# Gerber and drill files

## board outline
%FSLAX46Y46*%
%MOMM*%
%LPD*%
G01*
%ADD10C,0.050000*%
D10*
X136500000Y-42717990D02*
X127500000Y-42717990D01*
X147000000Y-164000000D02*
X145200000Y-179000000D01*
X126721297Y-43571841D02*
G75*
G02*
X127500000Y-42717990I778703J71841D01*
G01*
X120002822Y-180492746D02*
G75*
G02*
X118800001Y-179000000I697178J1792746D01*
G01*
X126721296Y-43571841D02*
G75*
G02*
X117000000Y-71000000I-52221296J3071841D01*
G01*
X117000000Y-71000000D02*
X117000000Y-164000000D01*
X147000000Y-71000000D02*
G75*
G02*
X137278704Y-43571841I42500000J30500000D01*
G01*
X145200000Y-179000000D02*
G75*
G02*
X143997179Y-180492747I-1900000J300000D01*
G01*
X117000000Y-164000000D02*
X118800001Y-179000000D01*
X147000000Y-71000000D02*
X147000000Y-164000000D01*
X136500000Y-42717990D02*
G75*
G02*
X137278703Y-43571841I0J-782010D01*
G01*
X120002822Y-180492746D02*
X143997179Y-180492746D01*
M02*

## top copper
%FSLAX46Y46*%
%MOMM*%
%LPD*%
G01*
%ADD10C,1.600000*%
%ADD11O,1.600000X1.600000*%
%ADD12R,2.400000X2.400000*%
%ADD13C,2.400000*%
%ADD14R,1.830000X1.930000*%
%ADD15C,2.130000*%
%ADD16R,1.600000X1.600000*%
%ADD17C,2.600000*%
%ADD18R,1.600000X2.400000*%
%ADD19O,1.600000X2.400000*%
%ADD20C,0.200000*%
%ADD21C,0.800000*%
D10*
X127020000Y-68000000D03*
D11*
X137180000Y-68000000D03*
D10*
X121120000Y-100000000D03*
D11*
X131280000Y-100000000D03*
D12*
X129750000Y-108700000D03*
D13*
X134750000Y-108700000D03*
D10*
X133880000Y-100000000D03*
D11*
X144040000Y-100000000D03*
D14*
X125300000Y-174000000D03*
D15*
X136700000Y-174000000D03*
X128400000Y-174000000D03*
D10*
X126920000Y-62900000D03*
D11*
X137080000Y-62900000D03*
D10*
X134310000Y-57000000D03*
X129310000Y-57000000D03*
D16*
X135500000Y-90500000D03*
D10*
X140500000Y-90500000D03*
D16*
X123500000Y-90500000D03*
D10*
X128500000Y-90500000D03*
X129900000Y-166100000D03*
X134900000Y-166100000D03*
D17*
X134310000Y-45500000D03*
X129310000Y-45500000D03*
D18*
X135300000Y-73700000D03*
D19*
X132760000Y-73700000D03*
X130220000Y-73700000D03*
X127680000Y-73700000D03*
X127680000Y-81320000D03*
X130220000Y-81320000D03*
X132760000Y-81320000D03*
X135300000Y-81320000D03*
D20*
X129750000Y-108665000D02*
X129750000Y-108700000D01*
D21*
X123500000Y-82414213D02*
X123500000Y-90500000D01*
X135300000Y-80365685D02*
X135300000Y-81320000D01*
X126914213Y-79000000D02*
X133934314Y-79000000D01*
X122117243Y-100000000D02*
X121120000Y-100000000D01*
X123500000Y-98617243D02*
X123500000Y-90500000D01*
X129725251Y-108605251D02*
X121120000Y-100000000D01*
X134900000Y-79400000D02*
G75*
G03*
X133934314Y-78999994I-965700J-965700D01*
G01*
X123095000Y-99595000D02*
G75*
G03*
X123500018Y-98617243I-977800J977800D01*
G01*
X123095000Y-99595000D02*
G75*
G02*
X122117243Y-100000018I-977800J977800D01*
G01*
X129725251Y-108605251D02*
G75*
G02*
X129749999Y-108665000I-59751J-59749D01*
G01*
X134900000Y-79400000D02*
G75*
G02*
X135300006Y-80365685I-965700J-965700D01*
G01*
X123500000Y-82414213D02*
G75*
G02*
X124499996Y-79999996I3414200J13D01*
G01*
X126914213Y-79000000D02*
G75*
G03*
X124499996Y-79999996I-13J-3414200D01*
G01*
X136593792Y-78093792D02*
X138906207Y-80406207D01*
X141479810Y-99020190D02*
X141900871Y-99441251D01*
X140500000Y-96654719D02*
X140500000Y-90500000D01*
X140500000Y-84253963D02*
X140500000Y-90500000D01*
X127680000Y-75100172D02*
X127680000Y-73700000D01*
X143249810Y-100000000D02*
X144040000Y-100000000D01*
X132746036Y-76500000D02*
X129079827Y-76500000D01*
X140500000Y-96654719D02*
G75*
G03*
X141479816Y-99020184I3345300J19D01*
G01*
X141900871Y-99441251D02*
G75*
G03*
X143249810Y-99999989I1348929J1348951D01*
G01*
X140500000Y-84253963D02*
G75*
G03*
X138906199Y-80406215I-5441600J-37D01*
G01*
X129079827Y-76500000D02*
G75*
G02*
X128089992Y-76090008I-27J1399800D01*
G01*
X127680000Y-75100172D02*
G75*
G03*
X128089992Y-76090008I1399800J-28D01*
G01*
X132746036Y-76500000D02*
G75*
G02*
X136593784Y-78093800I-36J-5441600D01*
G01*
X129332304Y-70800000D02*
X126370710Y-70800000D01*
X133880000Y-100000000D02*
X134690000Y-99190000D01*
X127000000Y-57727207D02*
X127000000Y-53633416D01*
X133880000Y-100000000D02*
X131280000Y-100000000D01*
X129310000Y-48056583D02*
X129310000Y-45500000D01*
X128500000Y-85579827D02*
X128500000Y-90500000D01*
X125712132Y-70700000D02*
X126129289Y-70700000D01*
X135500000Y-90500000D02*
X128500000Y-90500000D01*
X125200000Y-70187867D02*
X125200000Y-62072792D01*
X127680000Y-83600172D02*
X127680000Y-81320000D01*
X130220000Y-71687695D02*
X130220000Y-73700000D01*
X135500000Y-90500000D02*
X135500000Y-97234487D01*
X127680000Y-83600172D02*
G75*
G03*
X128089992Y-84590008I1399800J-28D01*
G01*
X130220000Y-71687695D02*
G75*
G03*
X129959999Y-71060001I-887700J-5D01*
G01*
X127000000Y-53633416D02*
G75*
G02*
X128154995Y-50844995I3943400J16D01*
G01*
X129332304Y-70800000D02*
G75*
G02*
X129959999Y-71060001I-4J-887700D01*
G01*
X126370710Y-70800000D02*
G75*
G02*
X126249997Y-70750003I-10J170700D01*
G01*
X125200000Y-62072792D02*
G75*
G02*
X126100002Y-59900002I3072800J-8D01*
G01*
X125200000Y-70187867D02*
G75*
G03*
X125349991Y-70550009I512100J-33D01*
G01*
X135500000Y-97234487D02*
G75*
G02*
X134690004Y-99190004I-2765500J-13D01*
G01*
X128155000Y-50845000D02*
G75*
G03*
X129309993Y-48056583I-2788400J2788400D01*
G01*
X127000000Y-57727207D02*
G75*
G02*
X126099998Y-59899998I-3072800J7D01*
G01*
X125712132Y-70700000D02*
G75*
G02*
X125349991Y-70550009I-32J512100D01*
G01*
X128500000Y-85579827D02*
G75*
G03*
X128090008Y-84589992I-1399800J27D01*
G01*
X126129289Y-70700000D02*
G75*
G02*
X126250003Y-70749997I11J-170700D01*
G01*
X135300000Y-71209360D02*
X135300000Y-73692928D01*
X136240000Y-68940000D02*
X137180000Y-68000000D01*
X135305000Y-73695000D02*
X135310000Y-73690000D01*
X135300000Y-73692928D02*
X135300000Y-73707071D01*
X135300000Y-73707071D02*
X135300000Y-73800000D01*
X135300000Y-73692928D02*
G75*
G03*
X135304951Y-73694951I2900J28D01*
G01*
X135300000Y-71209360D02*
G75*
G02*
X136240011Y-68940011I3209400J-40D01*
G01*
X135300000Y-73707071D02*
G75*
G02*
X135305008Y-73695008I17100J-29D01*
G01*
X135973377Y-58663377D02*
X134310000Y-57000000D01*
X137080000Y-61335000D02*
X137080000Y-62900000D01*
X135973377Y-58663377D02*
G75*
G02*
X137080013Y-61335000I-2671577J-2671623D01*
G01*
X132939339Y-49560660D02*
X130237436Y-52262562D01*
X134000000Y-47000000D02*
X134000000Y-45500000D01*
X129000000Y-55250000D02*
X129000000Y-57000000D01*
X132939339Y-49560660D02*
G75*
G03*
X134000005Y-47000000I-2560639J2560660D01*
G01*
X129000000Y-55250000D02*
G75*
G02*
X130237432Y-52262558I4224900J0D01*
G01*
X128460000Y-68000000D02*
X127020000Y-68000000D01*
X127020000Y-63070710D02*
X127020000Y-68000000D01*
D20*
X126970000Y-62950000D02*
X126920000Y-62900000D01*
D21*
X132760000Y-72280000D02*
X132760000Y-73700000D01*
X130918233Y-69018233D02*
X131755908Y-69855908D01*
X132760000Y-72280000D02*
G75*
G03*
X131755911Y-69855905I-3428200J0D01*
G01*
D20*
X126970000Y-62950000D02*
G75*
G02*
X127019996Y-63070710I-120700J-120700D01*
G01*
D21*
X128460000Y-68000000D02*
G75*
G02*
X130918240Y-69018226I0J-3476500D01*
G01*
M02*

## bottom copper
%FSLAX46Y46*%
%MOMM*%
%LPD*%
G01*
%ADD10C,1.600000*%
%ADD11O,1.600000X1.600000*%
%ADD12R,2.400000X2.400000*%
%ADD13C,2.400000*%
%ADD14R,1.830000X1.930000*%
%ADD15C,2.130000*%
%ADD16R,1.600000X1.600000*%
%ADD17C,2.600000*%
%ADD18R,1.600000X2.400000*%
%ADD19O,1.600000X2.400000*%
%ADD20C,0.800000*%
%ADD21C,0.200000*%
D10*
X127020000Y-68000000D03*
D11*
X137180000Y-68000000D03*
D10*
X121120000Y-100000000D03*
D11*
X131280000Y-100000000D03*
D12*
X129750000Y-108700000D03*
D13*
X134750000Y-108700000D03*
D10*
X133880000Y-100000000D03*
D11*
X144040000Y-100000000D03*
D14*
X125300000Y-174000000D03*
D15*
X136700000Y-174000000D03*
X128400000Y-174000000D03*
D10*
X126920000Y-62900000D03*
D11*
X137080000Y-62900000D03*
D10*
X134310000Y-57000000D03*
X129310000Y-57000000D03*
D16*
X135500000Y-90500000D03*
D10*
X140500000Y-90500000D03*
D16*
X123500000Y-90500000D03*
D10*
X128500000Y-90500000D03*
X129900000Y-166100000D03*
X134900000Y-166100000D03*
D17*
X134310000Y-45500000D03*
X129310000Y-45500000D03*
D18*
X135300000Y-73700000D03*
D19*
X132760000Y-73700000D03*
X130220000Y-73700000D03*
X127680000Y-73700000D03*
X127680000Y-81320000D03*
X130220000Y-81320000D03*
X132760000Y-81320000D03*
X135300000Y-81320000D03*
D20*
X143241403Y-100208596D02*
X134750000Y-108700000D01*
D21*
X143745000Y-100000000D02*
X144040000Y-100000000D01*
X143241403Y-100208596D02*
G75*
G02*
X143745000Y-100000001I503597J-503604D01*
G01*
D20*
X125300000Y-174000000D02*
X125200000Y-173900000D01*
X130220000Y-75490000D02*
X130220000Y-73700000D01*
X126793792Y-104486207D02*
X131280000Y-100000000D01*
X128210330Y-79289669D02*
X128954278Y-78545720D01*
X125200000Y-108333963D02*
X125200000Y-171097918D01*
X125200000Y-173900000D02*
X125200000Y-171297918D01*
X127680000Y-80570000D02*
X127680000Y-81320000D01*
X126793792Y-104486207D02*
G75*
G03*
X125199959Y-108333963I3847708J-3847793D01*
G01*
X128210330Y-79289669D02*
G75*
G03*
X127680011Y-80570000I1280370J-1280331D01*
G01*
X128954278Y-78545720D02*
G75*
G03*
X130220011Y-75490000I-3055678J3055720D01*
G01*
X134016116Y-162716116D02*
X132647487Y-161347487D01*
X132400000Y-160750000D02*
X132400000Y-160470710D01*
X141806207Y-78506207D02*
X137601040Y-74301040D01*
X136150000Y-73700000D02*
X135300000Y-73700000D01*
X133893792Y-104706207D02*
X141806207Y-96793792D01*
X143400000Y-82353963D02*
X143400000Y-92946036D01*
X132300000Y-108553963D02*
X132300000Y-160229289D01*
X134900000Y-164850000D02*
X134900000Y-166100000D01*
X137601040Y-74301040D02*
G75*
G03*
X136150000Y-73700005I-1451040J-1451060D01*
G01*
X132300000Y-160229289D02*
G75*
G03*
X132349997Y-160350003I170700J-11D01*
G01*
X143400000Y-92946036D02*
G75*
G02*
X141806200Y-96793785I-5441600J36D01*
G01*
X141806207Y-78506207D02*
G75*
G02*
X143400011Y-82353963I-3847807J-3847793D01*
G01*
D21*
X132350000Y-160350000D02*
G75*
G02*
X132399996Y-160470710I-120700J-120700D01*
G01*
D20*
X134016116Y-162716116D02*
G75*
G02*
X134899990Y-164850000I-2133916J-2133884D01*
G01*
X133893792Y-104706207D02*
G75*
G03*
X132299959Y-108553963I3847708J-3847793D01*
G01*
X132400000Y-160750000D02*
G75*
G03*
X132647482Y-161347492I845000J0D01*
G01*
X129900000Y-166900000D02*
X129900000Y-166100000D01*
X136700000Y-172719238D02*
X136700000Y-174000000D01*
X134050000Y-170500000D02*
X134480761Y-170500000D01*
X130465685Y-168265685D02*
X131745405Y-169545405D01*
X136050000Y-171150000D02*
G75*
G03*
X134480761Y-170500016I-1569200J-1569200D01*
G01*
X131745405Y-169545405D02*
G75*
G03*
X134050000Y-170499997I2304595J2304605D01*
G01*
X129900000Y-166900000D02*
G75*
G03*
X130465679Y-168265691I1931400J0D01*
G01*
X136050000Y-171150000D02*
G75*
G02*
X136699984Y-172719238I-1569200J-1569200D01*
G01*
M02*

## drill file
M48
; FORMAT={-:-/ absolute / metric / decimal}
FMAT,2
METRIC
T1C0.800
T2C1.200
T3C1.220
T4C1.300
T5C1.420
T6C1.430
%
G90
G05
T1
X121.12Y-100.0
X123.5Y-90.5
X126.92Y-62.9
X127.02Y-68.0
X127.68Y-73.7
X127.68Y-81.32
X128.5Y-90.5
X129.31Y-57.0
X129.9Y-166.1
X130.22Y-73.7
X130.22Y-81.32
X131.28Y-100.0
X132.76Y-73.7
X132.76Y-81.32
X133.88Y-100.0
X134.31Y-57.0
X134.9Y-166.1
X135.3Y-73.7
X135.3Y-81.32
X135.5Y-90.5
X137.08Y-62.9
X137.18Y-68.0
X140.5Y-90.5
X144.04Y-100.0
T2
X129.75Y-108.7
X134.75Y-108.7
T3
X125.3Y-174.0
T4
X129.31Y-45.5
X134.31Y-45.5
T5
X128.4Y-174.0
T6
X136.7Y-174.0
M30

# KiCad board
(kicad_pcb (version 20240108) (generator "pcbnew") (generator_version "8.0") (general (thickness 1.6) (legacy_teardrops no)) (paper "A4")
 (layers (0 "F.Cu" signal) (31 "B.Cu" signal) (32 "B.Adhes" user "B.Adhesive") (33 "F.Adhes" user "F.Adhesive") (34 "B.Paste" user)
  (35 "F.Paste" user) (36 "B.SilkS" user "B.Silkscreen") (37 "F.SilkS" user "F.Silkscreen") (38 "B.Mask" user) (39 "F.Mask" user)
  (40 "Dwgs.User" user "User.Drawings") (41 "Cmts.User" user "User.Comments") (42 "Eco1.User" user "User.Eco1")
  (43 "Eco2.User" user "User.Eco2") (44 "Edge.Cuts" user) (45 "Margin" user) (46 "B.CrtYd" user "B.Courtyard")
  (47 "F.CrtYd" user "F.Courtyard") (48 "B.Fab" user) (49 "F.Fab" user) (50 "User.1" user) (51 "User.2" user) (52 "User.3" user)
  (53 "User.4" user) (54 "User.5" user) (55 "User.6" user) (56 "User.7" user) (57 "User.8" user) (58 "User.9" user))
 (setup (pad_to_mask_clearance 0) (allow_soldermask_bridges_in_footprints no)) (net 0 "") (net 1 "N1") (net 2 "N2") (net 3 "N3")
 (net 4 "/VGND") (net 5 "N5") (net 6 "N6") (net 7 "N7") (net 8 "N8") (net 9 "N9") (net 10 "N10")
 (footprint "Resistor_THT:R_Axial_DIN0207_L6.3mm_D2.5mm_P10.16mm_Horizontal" (layer "F.Cu") (at 127.02 68)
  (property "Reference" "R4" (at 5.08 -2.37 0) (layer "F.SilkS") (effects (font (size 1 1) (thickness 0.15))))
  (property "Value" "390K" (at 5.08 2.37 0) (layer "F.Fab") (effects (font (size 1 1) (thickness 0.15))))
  (pad "1" thru_hole circle (at 0 0) (size 1.6 1.6) (drill 0.8) (layers "*.Cu" "*.Mask") (remove_unused_layers no) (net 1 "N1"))
  (pad "2" thru_hole oval (at 10.16 0) (size 1.6 1.6) (drill 0.8) (layers "*.Cu" "*.Mask") (remove_unused_layers no) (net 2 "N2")))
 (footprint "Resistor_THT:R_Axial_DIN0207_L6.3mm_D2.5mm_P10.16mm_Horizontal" (layer "F.Cu") (at 121.12 100)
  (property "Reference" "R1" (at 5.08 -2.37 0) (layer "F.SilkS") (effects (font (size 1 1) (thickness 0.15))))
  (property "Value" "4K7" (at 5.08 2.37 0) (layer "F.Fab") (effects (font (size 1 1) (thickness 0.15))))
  (pad "1" thru_hole circle (at 0 0) (size 1.6 1.6) (drill 0.8) (layers "*.Cu" "*.Mask") (remove_unused_layers no) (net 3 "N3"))
  (pad "2" thru_hole oval (at 10.16 0) (size 1.6 1.6) (drill 0.8) (layers "*.Cu" "*.Mask") (remove_unused_layers no) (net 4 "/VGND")))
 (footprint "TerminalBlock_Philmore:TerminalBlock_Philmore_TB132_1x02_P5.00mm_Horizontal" (layer "F.Cu") (at 129.75 108.7)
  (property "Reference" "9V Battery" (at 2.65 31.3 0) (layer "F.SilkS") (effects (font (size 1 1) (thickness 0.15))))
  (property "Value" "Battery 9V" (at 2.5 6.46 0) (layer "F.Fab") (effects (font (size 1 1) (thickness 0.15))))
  (pad "1" thru_hole rect (at 0 0) (size 2.4 2.4) (drill 1.2) (layers "*.Cu" "*.Mask") (remove_unused_layers no) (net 3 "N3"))
  (pad "2" thru_hole circle (at 5 0) (size 2.4 2.4) (drill 1.2) (layers "*.Cu" "*.Mask") (remove_unused_layers no) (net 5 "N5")))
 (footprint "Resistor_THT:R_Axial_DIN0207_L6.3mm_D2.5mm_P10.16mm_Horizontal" (layer "F.Cu") (at 133.88 100)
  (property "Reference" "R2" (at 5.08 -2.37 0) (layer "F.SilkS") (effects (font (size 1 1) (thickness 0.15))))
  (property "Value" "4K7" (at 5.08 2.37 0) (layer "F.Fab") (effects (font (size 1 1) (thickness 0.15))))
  (pad "1" thru_hole circle (at 0 0) (size 1.6 1.6) (drill 0.8) (layers "*.Cu" "*.Mask") (remove_unused_layers no) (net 4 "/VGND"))
  (pad "2" thru_hole oval (at 10.16 0) (size 1.6 1.6) (drill 0.8) (layers "*.Cu" "*.Mask") (remove_unused_layers no) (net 5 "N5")))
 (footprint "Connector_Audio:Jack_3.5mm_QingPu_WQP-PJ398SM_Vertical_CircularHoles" (layer "F.Cu") (at 125.3 174 90)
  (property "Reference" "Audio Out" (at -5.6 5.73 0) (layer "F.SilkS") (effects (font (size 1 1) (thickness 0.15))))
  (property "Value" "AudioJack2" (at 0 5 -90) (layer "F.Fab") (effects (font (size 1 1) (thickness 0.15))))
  (pad "S" thru_hole rect (at 0 0 270) (size 1.93 1.83) (drill 1.22) (layers "*.Cu" "*.Mask") (remove_unused_layers no) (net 4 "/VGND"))
  (pad "T" thru_hole circle (at 0 11.4 270) (size 2.13 2.13) (drill 1.43) (layers "*.Cu" "*.Mask") (remove_unused_layers no) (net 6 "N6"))
  (pad "TN" thru_hole circle (at 0 3.1 270) (size 2.13 2.13) (drill 1.42) (layers "*.Cu" "*.Mask") (remove_unused_layers no))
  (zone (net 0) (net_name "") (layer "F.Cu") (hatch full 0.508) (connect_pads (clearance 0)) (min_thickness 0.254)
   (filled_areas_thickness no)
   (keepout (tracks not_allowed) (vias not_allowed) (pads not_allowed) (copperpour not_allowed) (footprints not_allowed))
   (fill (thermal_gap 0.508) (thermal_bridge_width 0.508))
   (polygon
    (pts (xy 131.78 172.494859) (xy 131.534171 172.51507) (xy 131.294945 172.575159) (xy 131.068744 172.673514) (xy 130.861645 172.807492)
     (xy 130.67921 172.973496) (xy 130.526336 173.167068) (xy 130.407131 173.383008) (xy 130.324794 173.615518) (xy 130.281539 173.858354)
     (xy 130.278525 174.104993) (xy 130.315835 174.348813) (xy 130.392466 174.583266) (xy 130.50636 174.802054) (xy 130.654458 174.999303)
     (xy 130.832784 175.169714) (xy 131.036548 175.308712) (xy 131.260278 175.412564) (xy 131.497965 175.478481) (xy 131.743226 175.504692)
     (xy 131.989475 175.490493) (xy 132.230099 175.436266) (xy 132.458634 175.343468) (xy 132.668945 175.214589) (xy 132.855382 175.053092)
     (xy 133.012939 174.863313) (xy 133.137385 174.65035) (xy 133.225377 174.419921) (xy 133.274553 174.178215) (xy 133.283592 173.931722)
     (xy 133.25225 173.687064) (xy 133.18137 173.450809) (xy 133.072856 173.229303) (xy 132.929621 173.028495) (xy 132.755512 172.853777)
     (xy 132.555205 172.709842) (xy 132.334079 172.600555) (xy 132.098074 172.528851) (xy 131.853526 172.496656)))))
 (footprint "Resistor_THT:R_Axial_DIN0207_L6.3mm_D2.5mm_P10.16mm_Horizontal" (layer "F.Cu") (at 126.92 62.9)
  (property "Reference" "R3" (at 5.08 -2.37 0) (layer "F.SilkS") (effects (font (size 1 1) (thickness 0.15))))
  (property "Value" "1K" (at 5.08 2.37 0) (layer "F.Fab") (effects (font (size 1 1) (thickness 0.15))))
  (pad "1" thru_hole circle (at 0 0) (size 1.6 1.6) (drill 0.8) (layers "*.Cu" "*.Mask") (remove_unused_layers no) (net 1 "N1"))
  (pad "2" thru_hole oval (at 10.16 0) (size 1.6 1.6) (drill 0.8) (layers "*.Cu" "*.Mask") (remove_unused_layers no) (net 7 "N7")))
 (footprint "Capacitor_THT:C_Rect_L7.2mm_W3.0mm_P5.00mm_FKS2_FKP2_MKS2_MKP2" (layer "F.Cu") (at 134.31 57 180)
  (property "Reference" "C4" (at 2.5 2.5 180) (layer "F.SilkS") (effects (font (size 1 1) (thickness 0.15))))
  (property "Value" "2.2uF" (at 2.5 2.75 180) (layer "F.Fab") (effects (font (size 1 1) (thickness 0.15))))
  (pad "1" thru_hole circle (at 0 0 180) (size 1.6 1.6) (drill 0.8) (layers "*.Cu" "*.Mask") (remove_unused_layers no) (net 7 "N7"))
  (pad "2" thru_hole circle (at 5 0 180) (size 1.6 1.6) (drill 0.8) (layers "*.Cu" "*.Mask") (remove_unused_layers no) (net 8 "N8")))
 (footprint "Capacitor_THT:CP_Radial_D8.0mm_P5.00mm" (layer "F.Cu") (at 135.5 90.5)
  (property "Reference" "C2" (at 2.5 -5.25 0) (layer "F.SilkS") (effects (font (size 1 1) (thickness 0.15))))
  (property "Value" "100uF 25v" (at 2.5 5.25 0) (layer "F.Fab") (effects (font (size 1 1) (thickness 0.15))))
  (pad "1" thru_hole rect (at 0 0) (size 1.6 1.6) (drill 0.8) (layers "*.Cu" "*.Mask") (remove_unused_layers no) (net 4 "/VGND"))
  (pad "2" thru_hole circle (at 5 0) (size 1.6 1.6) (drill 0.8) (layers "*.Cu" "*.Mask") (remove_unused_layers no) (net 5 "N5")))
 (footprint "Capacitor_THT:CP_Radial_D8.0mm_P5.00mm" (layer "F.Cu") (at 123.5 90.5)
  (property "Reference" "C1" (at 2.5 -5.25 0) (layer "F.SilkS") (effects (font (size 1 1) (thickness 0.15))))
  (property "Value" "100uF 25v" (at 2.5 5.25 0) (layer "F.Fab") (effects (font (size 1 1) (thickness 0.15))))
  (pad "1" thru_hole rect (at 0 0) (size 1.6 1.6) (drill 0.8) (layers "*.Cu" "*.Mask") (remove_unused_layers no) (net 3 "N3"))
  (pad "2" thru_hole circle (at 5 0) (size 1.6 1.6) (drill 0.8) (layers "*.Cu" "*.Mask") (remove_unused_layers no) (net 4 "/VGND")))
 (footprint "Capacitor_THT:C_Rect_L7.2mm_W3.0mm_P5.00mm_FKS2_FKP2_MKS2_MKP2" (layer "F.Cu") (at 129.9 166.1)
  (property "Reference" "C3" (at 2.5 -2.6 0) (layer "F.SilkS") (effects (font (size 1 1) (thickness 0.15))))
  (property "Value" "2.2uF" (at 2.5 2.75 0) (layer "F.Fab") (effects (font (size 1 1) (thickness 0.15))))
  (pad "1" thru_hole circle (at 0 0) (size 1.6 1.6) (drill 0.8) (layers "*.Cu" "*.Mask") (remove_unused_layers no) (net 6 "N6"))
  (pad "2" thru_hole circle (at 5 0) (size 1.6 1.6) (drill 0.8) (layers "*.Cu" "*.Mask") (remove_unused_layers no) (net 2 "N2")))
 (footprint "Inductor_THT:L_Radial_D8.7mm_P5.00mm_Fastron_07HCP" (layer "F.Cu") (at 134.31 45.5 180)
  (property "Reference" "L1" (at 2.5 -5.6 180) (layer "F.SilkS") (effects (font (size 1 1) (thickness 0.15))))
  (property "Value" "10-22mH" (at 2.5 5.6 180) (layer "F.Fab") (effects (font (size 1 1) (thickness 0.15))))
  (pad "1" thru_hole circle (at 0 0 180) (size 2.6 2.6) (drill 1.3) (layers "*.Cu" "*.Mask") (remove_unused_layers no) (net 8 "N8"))
  (pad "2" thru_hole circle (at 5 0 180) (size 2.6 2.6) (drill 1.3) (layers "*.Cu" "*.Mask") (remove_unused_layers no) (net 4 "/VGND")))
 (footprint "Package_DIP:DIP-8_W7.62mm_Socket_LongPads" (layer "F.Cu") (at 135.3 73.7 -90)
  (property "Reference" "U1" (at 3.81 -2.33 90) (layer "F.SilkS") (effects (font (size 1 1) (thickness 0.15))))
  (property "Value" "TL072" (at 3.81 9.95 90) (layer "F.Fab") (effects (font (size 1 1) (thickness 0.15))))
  (pad "1" thru_hole rect (at 0 0 270) (size 2.4 1.6) (drill 0.8) (layers "*.Cu" "*.Mask") (remove_unused_layers no) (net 2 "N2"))
  (pad "2" thru_hole oval (at 0 2.54 270) (size 2.4 1.6) (drill 0.8) (layers "*.Cu" "*.Mask") (remove_unused_layers no) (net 1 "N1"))
  (pad "3" thru_hole oval (at 0 5.08 270) (size 2.4 1.6) (drill 0.8) (layers "*.Cu" "*.Mask") (remove_unused_layers no) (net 4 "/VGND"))
  (pad "4" thru_hole oval (at 0 7.62 270) (size 2.4 1.6) (drill 0.8) (layers "*.Cu" "*.Mask") (remove_unused_layers no) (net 5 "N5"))
  (pad "5" thru_hole oval (at 7.62 7.62 270) (size 2.4 1.6) (drill 0.8) (layers "*.Cu" "*.Mask") (remove_unused_layers no) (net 4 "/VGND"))
  (pad "6" thru_hole oval (at 7.62 5.08 270) (size 2.4 1.6) (drill 0.8) (layers "*.Cu" "*.Mask") (remove_unused_layers no) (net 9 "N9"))
  (pad "7" thru_hole oval (at 7.62 2.54 270) (size 2.4 1.6) (drill 0.8) (layers "*.Cu" "*.Mask") (remove_unused_layers no) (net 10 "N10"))
  (pad "8" thru_hole oval (at 7.62 0 270) (size 2.4 1.6) (drill 0.8) (layers "*.Cu" "*.Mask") (remove_unused_layers no) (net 3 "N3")))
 (gr_line (start 136.5 42.71799) (end 127.5 42.71799) (stroke (width 0.05) (type default)) (layer "Edge.Cuts"))
 (gr_line (start 147 164) (end 145.2 179) (stroke (width 0.05) (type default)) (layer "Edge.Cuts"))
 (gr_arc (start 126.721297 43.571841) (mid 126.922194 42.973047) (end 127.5 42.71799) (stroke (width 0.05) (type default))
  (layer "Edge.Cuts"))
 (gr_arc (start 120.002822 180.492746) (mid 119.2022 179.906893) (end 118.800001 179) (stroke (width 0.05) (type default))
  (layer "Edge.Cuts"))
 (gr_arc (start 126.721296 43.571841) (mid 123.806256 57.975497) (end 117 71) (stroke (width 0.05) (type default)) (layer "Edge.Cuts"))
 (gr_line (start 117 71) (end 117 164) (stroke (width 0.05) (type default)) (layer "Edge.Cuts"))
 (gr_arc (start 147 71) (mid 140.193743 57.975498) (end 137.278704 43.571841) (stroke (width 0.05) (type default)) (layer "Edge.Cuts"))
 (gr_arc (start 145.2 179) (mid 144.797801 179.906893) (end 143.997179 180.492746) (stroke (width 0.05) (type default)) (layer "Edge.Cuts"))
 (gr_line (start 117 164) (end 118.800001 179) (stroke (width 0.05) (type default)) (layer "Edge.Cuts"))
 (gr_line (start 147 71) (end 147 164) (stroke (width 0.05) (type default)) (layer "Edge.Cuts"))
 (gr_arc (start 136.5 42.71799) (mid 137.077806 42.973047) (end 137.278703 43.571841) (stroke (width 0.05) (type default))
  (layer "Edge.Cuts"))
 (gr_line (start 120.002822 180.492746) (end 143.997179 180.492746) (stroke (width 0.05) (type default)) (layer "Edge.Cuts"))
 (segment (start 129.75 108.665) (end 129.75 108.7) (width 0.2) (layer "F.Cu") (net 3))
 (segment (start 123.5 82.414213) (end 123.5 90.5) (width 0.8) (layer "F.Cu") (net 3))
 (segment (start 135.3 80.365685) (end 135.3 81.32) (width 0.8) (layer "F.Cu") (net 3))
 (segment (start 126.914213 79) (end 133.934314 79) (width 0.8) (layer "F.Cu") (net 3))
 (segment (start 122.117243 100) (end 121.12 100) (width 0.8) (layer "F.Cu") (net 3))
 (segment (start 123.5 98.617243) (end 123.5 90.5) (width 0.8) (layer "F.Cu") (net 3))
 (segment (start 129.725251 108.605251) (end 121.12 100) (width 0.8) (layer "F.Cu") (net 3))
 (arc (start 134.9 79.4) (mid 134.456939 79.103956) (end 133.934314 79) (width 0.8) (layer "F.Cu") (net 3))
 (arc (start 123.095 99.595) (mid 123.394743 99.146401) (end 123.5 98.617243) (width 0.8) (layer "F.Cu") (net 3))
 (arc (start 123.095 99.595) (mid 122.646401 99.894743) (end 122.117243 100) (width 0.8) (layer "F.Cu") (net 3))
 (arc (start 129.725251 108.605251) (mid 129.743567 108.632664) (end 129.75 108.665) (width 0.8) (layer "F.Cu") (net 3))
 (arc (start 134.9 79.4) (mid 135.196043 79.84306) (end 135.3 80.365685) (width 0.8) (layer "F.Cu") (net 3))
 (arc (start 123.5 82.414213) (mid 123.759891 81.10765) (end 124.5 80) (width 0.8) (layer "F.Cu") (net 3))
 (arc (start 126.914213 79) (mid 125.60765 79.259891) (end 124.5 80) (width 0.8) (layer "F.Cu") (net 3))
 (segment (start 136.593792 78.093792) (end 138.906207 80.406207) (width 0.8) (layer "F.Cu") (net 5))
 (segment (start 141.47981 99.02019) (end 141.900871 99.441251) (width 0.8) (layer "F.Cu") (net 5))
 (segment (start 140.5 96.654719) (end 140.5 90.5) (width 0.8) (layer "F.Cu") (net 5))
 (segment (start 140.5 84.253963) (end 140.5 90.5) (width 0.8) (layer "F.Cu") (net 5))
 (segment (start 127.68 75.100172) (end 127.68 73.7) (width 0.8) (layer "F.Cu") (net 5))
 (segment (start 143.24981 100) (end 144.04 100) (width 0.8) (layer "F.Cu") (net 5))
 (segment (start 132.746036 76.5) (end 129.079827 76.5) (width 0.8) (layer "F.Cu") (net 5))
 (arc (start 140.5 96.654719) (mid 140.754644 97.934902) (end 141.47981 99.02019) (width 0.8) (layer "F.Cu") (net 5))
 (arc (start 141.900871 99.441251) (mid 142.519769 99.854785) (end 143.24981 100) (width 0.8) (layer "F.Cu") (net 5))
 (arc (start 140.5 84.253963) (mid 140.085786 82.171572) (end 138.906207 80.406207) (width 0.8) (layer "F.Cu") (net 5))
 (arc (start 129.079827 76.5) (mid 128.544136 76.393444) (end 128.09 76.09) (width 0.8) (layer "F.Cu") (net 5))
 (arc (start 127.68 75.100172) (mid 127.786555 75.635863) (end 128.09 76.09) (width 0.8) (layer "F.Cu") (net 5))
 (arc (start 132.746036 76.5) (mid 134.828426 76.914213) (end 136.593792 78.093792) (width 0.8) (layer "F.Cu") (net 5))
 (segment (start 143.241403 100.208596) (end 134.75 108.7) (width 0.8) (layer "B.Cu") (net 5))
 (segment (start 143.745 100) (end 144.04 100) (width 0.2) (layer "B.Cu") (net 5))
 (arc (start 143.241403 100.208596) (mid 143.472455 100.054212) (end 143.745 100) (width 0.2) (layer "B.Cu") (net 5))
 (segment (start 129.332304 70.8) (end 126.37071 70.8) (width 0.8) (layer "F.Cu") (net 4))
 (segment (start 133.88 100) (end 134.69 99.19) (width 0.8) (layer "F.Cu") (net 4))
 (segment (start 127 57.727207) (end 127 53.633416) (width 0.8) (layer "F.Cu") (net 4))
 (segment (start 133.88 100) (end 131.28 100) (width 0.8) (layer "F.Cu") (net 4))
 (segment (start 129.31 48.056583) (end 129.31 45.5) (width 0.8) (layer "F.Cu") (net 4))
 (segment (start 128.5 85.579827) (end 128.5 90.5) (width 0.8) (layer "F.Cu") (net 4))
 (segment (start 125.712132 70.7) (end 126.129289 70.7) (width 0.8) (layer "F.Cu") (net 4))
 (segment (start 135.5 90.5) (end 128.5 90.5) (width 0.8) (layer "F.Cu") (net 4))
 (segment (start 125.2 70.187867) (end 125.2 62.072792) (width 0.8) (layer "F.Cu") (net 4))
 (segment (start 127.68 83.600172) (end 127.68 81.32) (width 0.8) (layer "F.Cu") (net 4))
 (segment (start 130.22 71.687695) (end 130.22 73.7) (width 0.8) (layer "F.Cu") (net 4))
 (segment (start 135.5 90.5) (end 135.5 97.234487) (width 0.8) (layer "F.Cu") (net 4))
 (arc (start 127.68 83.600172) (mid 127.786555 84.135863) (end 128.09 84.59) (width 0.8) (layer "F.Cu") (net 4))
 (arc (start 130.22 71.687695) (mid 130.152428 71.347989) (end 129.96 71.06) (width 0.8) (layer "F.Cu") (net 4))
 (arc (start 127 53.633416) (mid 127.300174 52.124336) (end 128.155 50.845) (width 0.8) (layer "F.Cu") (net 4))
 (arc (start 129.332304 70.8) (mid 129.67201 70.867571) (end 129.96 71.06) (width 0.8) (layer "F.Cu") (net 4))
 (arc (start 126.37071 70.8) (mid 126.305382 70.787005) (end 126.25 70.75) (width 0.8) (layer "F.Cu") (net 4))
 (arc (start 125.2 62.072792) (mid 125.433902 60.896885) (end 126.1 59.9) (width 0.8) (layer "F.Cu") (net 4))
 (arc (start 125.2 70.187867) (mid 125.238983 70.383852) (end 125.35 70.55) (width 0.8) (layer "F.Cu") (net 4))
 (arc (start 135.5 97.234487) (mid 135.289487 98.292803) (end 134.69 99.19) (width 0.8) (layer "F.Cu") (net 4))
 (arc (start 128.155 50.845) (mid 129.009825 49.565663) (end 129.31 48.056583) (width 0.8) (layer "F.Cu") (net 4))
 (arc (start 127 57.727207) (mid 126.766097 58.903114) (end 126.1 59.9) (width 0.8) (layer "F.Cu") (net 4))
 (arc (start 125.712132 70.7) (mid 125.516147 70.661016) (end 125.35 70.55) (width 0.8) (layer "F.Cu") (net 4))
 (arc (start 128.5 85.579827) (mid 128.393444 85.044136) (end 128.09 84.59) (width 0.8) (layer "F.Cu") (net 4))
 (arc (start 126.129289 70.7) (mid 126.194617 70.712994) (end 126.25 70.75) (width 0.8) (layer "F.Cu") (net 4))
 (segment (start 125.3 174) (end 125.2 173.9) (width 0.8) (layer "B.Cu") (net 4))
 (segment (start 130.22 75.49) (end 130.22 73.7) (width 0.8) (layer "B.Cu") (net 4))
 (segment (start 126.793792 104.486207) (end 131.28 100) (width 0.8) (layer "B.Cu") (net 4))
 (segment (start 128.21033 79.289669) (end 128.954278 78.54572) (width 0.8) (layer "B.Cu") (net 4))
 (segment (start 125.2 108.333963) (end 125.2 171.097918) (width 0.8) (layer "B.Cu") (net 4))
 (segment (start 125.2 173.9) (end 125.2 171.297918) (width 0.8) (layer "B.Cu") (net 4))
 (segment (start 127.68 80.57) (end 127.68 81.32) (width 0.8) (layer "B.Cu") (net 4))
 (arc (start 126.793792 104.486207) (mid 125.614213 106.251572) (end 125.2 108.333963) (width 0.8) (layer "B.Cu") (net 4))
 (arc (start 128.21033 79.289669) (mid 127.817828 79.87709) (end 127.68 80.57) (width 0.8) (layer "B.Cu") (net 4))
 (arc (start 128.954278 78.54572) (mid 129.891049 77.143744) (end 130.22 75.49) (width 0.8) (layer "B.Cu") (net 4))
 (segment (start 135.3 71.20936) (end 135.3 73.692928) (width 0.8) (layer "F.Cu") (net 2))
 (segment (start 136.24 68.94) (end 137.18 68) (width 0.8) (layer "F.Cu") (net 2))
 (segment (start 135.305 73.695) (end 135.31 73.69) (width 0.8) (layer "F.Cu") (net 2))
 (segment (start 135.3 73.692928) (end 135.3 73.707071) (width 0.8) (layer "F.Cu") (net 2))
 (segment (start 135.3 73.707071) (end 135.3 73.8) (width 0.8) (layer "F.Cu") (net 2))
 (arc (start 135.3 73.692928) (mid 135.301808 73.695634) (end 135.305 73.695) (width 0.8) (layer "F.Cu") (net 2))
 (arc (start 135.3 71.20936) (mid 135.544298 69.981191) (end 136.24 68.94) (width 0.8) (layer "F.Cu") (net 2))
 (arc (start 135.3 73.707071) (mid 135.301299 73.700538) (end 135.305 73.695) (width 0.8) (layer "F.Cu") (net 2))
 (segment (start 134.016116 162.716116) (end 132.647487 161.347487) (width 0.8) (layer "B.Cu") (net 2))
 (segment (start 132.4 160.75) (end 132.4 160.47071) (width 0.8) (layer "B.Cu") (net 2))
 (segment (start 141.806207 78.506207) (end 137.60104 74.30104) (width 0.8) (layer "B.Cu") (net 2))
 (segment (start 136.15 73.7) (end 135.3 73.7) (width 0.8) (layer "B.Cu") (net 2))
 (segment (start 133.893792 104.706207) (end 141.806207 96.793792) (width 0.8) (layer "B.Cu") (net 2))
 (segment (start 143.4 82.353963) (end 143.4 92.946036) (width 0.8) (layer "B.Cu") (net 2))
 (segment (start 132.3 108.553963) (end 132.3 160.229289) (width 0.8) (layer "B.Cu") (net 2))
 (segment (start 134.9 164.85) (end 134.9 166.1) (width 0.8) (layer "B.Cu") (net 2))
 (arc (start 137.60104 74.30104) (mid 136.935297 73.856205) (end 136.15 73.7) (width 0.8) (layer "B.Cu") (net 2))
 (arc (start 132.3 160.229289) (mid 132.312994 160.294617) (end 132.35 160.35) (width 0.8) (layer "B.Cu") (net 2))
 (arc (start 143.4 92.946036) (mid 142.985786 95.028426) (end 141.806207 96.793792) (width 0.8) (layer "B.Cu") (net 2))
 (arc (start 141.806207 78.506207) (mid 142.985786 80.271572) (end 143.4 82.353963) (width 0.8) (layer "B.Cu") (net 2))
 (arc (start 132.35 160.35) (mid 132.387005 160.405382) (end 132.4 160.47071) (width 0.2) (layer "B.Cu") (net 2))
 (arc (start 134.016116 162.716116) (mid 134.670286 163.69515) (end 134.9 164.85) (width 0.8) (layer "B.Cu") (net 2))
 (arc (start 133.893792 104.706207) (mid 132.714213 106.471572) (end 132.3 108.553963) (width 0.8) (layer "B.Cu") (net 2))
 (arc (start 132.4 160.75) (mid 132.464319 161.073357) (end 132.647487 161.347487) (width 0.8) (layer "B.Cu") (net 2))
 (segment (start 129.9 166.9) (end 129.9 166.1) (width 0.8) (layer "B.Cu") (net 6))
 (segment (start 136.7 172.719238) (end 136.7 174) (width 0.8) (layer "B.Cu") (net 6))
 (segment (start 134.05 170.5) (end 134.480761 170.5) (width 0.8) (layer "B.Cu") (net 6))
 (segment (start 130.465685 168.265685) (end 131.745405 169.545405) (width 0.8) (layer "B.Cu") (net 6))
 (arc (start 136.05 171.15) (mid 135.330027 170.668929) (end 134.480761 170.5) (width 0.8) (layer "B.Cu") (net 6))
 (arc (start 131.745405 169.545405) (mid 132.802762 170.251908) (end 134.05 170.5) (width 0.8) (layer "B.Cu") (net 6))
 (arc (start 129.9 166.9) (mid 130.047016 167.639103) (end 130.465685 168.265685) (width 0.8) (layer "B.Cu") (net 6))
 (arc (start 136.05 171.15) (mid 136.53107 171.869972) (end 136.7 172.719238) (width 0.8) (layer "B.Cu") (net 6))
 (segment (start 135.973377 58.663377) (end 134.31 57) (width 0.8) (layer "F.Cu") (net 7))
 (segment (start 137.08 61.335) (end 137.08 62.9) (width 0.8) (layer "F.Cu") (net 7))
 (arc (start 135.973377 58.663377) (mid 136.792398 59.889128) (end 137.08 61.335) (width 0.8) (layer "F.Cu") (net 7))
 (segment (start 132.939339 49.56066) (end 130.237436 52.262562) (width 0.8) (layer "F.Cu") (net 8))
 (segment (start 134 47) (end 134 45.5) (width 0.8) (layer "F.Cu") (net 8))
 (segment (start 129 55.25) (end 129 57) (width 0.8) (layer "F.Cu") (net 8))
 (arc (start 132.939339 49.56066) (mid 133.724343 48.385819) (end 134 47) (width 0.8) (layer "F.Cu") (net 8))
 (arc (start 129 55.25) (mid 129.321599 53.63321) (end 130.237436 52.262562) (width 0.8) (layer "F.Cu") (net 8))
 (segment (start 128.46 68) (end 127.02 68) (width 0.8) (layer "F.Cu") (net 1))
 (segment (start 127.02 63.07071) (end 127.02 68) (width 0.8) (layer "F.Cu") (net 1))
 (segment (start 126.97 62.95) (end 126.92 62.9) (width 0.2) (layer "F.Cu") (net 1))
 (segment (start 132.76 72.28) (end 132.76 73.7) (width 0.8) (layer "F.Cu") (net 1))
 (segment (start 130.918233 69.018233) (end 131.755908 69.855908) (width 0.8) (layer "F.Cu") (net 1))
 (arc (start 132.76 72.28) (mid 132.499044 70.96809) (end 131.755908 69.855908) (width 0.8) (layer "F.Cu") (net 1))
 (arc (start 126.97 62.95) (mid 127.007005 63.005382) (end 127.02 63.07071) (width 0.2) (layer "F.Cu") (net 1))
 (arc (start 128.46 68) (mid 129.790386 68.26463) (end 130.918233 69.018233) (width 0.8) (layer "F.Cu") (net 1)))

